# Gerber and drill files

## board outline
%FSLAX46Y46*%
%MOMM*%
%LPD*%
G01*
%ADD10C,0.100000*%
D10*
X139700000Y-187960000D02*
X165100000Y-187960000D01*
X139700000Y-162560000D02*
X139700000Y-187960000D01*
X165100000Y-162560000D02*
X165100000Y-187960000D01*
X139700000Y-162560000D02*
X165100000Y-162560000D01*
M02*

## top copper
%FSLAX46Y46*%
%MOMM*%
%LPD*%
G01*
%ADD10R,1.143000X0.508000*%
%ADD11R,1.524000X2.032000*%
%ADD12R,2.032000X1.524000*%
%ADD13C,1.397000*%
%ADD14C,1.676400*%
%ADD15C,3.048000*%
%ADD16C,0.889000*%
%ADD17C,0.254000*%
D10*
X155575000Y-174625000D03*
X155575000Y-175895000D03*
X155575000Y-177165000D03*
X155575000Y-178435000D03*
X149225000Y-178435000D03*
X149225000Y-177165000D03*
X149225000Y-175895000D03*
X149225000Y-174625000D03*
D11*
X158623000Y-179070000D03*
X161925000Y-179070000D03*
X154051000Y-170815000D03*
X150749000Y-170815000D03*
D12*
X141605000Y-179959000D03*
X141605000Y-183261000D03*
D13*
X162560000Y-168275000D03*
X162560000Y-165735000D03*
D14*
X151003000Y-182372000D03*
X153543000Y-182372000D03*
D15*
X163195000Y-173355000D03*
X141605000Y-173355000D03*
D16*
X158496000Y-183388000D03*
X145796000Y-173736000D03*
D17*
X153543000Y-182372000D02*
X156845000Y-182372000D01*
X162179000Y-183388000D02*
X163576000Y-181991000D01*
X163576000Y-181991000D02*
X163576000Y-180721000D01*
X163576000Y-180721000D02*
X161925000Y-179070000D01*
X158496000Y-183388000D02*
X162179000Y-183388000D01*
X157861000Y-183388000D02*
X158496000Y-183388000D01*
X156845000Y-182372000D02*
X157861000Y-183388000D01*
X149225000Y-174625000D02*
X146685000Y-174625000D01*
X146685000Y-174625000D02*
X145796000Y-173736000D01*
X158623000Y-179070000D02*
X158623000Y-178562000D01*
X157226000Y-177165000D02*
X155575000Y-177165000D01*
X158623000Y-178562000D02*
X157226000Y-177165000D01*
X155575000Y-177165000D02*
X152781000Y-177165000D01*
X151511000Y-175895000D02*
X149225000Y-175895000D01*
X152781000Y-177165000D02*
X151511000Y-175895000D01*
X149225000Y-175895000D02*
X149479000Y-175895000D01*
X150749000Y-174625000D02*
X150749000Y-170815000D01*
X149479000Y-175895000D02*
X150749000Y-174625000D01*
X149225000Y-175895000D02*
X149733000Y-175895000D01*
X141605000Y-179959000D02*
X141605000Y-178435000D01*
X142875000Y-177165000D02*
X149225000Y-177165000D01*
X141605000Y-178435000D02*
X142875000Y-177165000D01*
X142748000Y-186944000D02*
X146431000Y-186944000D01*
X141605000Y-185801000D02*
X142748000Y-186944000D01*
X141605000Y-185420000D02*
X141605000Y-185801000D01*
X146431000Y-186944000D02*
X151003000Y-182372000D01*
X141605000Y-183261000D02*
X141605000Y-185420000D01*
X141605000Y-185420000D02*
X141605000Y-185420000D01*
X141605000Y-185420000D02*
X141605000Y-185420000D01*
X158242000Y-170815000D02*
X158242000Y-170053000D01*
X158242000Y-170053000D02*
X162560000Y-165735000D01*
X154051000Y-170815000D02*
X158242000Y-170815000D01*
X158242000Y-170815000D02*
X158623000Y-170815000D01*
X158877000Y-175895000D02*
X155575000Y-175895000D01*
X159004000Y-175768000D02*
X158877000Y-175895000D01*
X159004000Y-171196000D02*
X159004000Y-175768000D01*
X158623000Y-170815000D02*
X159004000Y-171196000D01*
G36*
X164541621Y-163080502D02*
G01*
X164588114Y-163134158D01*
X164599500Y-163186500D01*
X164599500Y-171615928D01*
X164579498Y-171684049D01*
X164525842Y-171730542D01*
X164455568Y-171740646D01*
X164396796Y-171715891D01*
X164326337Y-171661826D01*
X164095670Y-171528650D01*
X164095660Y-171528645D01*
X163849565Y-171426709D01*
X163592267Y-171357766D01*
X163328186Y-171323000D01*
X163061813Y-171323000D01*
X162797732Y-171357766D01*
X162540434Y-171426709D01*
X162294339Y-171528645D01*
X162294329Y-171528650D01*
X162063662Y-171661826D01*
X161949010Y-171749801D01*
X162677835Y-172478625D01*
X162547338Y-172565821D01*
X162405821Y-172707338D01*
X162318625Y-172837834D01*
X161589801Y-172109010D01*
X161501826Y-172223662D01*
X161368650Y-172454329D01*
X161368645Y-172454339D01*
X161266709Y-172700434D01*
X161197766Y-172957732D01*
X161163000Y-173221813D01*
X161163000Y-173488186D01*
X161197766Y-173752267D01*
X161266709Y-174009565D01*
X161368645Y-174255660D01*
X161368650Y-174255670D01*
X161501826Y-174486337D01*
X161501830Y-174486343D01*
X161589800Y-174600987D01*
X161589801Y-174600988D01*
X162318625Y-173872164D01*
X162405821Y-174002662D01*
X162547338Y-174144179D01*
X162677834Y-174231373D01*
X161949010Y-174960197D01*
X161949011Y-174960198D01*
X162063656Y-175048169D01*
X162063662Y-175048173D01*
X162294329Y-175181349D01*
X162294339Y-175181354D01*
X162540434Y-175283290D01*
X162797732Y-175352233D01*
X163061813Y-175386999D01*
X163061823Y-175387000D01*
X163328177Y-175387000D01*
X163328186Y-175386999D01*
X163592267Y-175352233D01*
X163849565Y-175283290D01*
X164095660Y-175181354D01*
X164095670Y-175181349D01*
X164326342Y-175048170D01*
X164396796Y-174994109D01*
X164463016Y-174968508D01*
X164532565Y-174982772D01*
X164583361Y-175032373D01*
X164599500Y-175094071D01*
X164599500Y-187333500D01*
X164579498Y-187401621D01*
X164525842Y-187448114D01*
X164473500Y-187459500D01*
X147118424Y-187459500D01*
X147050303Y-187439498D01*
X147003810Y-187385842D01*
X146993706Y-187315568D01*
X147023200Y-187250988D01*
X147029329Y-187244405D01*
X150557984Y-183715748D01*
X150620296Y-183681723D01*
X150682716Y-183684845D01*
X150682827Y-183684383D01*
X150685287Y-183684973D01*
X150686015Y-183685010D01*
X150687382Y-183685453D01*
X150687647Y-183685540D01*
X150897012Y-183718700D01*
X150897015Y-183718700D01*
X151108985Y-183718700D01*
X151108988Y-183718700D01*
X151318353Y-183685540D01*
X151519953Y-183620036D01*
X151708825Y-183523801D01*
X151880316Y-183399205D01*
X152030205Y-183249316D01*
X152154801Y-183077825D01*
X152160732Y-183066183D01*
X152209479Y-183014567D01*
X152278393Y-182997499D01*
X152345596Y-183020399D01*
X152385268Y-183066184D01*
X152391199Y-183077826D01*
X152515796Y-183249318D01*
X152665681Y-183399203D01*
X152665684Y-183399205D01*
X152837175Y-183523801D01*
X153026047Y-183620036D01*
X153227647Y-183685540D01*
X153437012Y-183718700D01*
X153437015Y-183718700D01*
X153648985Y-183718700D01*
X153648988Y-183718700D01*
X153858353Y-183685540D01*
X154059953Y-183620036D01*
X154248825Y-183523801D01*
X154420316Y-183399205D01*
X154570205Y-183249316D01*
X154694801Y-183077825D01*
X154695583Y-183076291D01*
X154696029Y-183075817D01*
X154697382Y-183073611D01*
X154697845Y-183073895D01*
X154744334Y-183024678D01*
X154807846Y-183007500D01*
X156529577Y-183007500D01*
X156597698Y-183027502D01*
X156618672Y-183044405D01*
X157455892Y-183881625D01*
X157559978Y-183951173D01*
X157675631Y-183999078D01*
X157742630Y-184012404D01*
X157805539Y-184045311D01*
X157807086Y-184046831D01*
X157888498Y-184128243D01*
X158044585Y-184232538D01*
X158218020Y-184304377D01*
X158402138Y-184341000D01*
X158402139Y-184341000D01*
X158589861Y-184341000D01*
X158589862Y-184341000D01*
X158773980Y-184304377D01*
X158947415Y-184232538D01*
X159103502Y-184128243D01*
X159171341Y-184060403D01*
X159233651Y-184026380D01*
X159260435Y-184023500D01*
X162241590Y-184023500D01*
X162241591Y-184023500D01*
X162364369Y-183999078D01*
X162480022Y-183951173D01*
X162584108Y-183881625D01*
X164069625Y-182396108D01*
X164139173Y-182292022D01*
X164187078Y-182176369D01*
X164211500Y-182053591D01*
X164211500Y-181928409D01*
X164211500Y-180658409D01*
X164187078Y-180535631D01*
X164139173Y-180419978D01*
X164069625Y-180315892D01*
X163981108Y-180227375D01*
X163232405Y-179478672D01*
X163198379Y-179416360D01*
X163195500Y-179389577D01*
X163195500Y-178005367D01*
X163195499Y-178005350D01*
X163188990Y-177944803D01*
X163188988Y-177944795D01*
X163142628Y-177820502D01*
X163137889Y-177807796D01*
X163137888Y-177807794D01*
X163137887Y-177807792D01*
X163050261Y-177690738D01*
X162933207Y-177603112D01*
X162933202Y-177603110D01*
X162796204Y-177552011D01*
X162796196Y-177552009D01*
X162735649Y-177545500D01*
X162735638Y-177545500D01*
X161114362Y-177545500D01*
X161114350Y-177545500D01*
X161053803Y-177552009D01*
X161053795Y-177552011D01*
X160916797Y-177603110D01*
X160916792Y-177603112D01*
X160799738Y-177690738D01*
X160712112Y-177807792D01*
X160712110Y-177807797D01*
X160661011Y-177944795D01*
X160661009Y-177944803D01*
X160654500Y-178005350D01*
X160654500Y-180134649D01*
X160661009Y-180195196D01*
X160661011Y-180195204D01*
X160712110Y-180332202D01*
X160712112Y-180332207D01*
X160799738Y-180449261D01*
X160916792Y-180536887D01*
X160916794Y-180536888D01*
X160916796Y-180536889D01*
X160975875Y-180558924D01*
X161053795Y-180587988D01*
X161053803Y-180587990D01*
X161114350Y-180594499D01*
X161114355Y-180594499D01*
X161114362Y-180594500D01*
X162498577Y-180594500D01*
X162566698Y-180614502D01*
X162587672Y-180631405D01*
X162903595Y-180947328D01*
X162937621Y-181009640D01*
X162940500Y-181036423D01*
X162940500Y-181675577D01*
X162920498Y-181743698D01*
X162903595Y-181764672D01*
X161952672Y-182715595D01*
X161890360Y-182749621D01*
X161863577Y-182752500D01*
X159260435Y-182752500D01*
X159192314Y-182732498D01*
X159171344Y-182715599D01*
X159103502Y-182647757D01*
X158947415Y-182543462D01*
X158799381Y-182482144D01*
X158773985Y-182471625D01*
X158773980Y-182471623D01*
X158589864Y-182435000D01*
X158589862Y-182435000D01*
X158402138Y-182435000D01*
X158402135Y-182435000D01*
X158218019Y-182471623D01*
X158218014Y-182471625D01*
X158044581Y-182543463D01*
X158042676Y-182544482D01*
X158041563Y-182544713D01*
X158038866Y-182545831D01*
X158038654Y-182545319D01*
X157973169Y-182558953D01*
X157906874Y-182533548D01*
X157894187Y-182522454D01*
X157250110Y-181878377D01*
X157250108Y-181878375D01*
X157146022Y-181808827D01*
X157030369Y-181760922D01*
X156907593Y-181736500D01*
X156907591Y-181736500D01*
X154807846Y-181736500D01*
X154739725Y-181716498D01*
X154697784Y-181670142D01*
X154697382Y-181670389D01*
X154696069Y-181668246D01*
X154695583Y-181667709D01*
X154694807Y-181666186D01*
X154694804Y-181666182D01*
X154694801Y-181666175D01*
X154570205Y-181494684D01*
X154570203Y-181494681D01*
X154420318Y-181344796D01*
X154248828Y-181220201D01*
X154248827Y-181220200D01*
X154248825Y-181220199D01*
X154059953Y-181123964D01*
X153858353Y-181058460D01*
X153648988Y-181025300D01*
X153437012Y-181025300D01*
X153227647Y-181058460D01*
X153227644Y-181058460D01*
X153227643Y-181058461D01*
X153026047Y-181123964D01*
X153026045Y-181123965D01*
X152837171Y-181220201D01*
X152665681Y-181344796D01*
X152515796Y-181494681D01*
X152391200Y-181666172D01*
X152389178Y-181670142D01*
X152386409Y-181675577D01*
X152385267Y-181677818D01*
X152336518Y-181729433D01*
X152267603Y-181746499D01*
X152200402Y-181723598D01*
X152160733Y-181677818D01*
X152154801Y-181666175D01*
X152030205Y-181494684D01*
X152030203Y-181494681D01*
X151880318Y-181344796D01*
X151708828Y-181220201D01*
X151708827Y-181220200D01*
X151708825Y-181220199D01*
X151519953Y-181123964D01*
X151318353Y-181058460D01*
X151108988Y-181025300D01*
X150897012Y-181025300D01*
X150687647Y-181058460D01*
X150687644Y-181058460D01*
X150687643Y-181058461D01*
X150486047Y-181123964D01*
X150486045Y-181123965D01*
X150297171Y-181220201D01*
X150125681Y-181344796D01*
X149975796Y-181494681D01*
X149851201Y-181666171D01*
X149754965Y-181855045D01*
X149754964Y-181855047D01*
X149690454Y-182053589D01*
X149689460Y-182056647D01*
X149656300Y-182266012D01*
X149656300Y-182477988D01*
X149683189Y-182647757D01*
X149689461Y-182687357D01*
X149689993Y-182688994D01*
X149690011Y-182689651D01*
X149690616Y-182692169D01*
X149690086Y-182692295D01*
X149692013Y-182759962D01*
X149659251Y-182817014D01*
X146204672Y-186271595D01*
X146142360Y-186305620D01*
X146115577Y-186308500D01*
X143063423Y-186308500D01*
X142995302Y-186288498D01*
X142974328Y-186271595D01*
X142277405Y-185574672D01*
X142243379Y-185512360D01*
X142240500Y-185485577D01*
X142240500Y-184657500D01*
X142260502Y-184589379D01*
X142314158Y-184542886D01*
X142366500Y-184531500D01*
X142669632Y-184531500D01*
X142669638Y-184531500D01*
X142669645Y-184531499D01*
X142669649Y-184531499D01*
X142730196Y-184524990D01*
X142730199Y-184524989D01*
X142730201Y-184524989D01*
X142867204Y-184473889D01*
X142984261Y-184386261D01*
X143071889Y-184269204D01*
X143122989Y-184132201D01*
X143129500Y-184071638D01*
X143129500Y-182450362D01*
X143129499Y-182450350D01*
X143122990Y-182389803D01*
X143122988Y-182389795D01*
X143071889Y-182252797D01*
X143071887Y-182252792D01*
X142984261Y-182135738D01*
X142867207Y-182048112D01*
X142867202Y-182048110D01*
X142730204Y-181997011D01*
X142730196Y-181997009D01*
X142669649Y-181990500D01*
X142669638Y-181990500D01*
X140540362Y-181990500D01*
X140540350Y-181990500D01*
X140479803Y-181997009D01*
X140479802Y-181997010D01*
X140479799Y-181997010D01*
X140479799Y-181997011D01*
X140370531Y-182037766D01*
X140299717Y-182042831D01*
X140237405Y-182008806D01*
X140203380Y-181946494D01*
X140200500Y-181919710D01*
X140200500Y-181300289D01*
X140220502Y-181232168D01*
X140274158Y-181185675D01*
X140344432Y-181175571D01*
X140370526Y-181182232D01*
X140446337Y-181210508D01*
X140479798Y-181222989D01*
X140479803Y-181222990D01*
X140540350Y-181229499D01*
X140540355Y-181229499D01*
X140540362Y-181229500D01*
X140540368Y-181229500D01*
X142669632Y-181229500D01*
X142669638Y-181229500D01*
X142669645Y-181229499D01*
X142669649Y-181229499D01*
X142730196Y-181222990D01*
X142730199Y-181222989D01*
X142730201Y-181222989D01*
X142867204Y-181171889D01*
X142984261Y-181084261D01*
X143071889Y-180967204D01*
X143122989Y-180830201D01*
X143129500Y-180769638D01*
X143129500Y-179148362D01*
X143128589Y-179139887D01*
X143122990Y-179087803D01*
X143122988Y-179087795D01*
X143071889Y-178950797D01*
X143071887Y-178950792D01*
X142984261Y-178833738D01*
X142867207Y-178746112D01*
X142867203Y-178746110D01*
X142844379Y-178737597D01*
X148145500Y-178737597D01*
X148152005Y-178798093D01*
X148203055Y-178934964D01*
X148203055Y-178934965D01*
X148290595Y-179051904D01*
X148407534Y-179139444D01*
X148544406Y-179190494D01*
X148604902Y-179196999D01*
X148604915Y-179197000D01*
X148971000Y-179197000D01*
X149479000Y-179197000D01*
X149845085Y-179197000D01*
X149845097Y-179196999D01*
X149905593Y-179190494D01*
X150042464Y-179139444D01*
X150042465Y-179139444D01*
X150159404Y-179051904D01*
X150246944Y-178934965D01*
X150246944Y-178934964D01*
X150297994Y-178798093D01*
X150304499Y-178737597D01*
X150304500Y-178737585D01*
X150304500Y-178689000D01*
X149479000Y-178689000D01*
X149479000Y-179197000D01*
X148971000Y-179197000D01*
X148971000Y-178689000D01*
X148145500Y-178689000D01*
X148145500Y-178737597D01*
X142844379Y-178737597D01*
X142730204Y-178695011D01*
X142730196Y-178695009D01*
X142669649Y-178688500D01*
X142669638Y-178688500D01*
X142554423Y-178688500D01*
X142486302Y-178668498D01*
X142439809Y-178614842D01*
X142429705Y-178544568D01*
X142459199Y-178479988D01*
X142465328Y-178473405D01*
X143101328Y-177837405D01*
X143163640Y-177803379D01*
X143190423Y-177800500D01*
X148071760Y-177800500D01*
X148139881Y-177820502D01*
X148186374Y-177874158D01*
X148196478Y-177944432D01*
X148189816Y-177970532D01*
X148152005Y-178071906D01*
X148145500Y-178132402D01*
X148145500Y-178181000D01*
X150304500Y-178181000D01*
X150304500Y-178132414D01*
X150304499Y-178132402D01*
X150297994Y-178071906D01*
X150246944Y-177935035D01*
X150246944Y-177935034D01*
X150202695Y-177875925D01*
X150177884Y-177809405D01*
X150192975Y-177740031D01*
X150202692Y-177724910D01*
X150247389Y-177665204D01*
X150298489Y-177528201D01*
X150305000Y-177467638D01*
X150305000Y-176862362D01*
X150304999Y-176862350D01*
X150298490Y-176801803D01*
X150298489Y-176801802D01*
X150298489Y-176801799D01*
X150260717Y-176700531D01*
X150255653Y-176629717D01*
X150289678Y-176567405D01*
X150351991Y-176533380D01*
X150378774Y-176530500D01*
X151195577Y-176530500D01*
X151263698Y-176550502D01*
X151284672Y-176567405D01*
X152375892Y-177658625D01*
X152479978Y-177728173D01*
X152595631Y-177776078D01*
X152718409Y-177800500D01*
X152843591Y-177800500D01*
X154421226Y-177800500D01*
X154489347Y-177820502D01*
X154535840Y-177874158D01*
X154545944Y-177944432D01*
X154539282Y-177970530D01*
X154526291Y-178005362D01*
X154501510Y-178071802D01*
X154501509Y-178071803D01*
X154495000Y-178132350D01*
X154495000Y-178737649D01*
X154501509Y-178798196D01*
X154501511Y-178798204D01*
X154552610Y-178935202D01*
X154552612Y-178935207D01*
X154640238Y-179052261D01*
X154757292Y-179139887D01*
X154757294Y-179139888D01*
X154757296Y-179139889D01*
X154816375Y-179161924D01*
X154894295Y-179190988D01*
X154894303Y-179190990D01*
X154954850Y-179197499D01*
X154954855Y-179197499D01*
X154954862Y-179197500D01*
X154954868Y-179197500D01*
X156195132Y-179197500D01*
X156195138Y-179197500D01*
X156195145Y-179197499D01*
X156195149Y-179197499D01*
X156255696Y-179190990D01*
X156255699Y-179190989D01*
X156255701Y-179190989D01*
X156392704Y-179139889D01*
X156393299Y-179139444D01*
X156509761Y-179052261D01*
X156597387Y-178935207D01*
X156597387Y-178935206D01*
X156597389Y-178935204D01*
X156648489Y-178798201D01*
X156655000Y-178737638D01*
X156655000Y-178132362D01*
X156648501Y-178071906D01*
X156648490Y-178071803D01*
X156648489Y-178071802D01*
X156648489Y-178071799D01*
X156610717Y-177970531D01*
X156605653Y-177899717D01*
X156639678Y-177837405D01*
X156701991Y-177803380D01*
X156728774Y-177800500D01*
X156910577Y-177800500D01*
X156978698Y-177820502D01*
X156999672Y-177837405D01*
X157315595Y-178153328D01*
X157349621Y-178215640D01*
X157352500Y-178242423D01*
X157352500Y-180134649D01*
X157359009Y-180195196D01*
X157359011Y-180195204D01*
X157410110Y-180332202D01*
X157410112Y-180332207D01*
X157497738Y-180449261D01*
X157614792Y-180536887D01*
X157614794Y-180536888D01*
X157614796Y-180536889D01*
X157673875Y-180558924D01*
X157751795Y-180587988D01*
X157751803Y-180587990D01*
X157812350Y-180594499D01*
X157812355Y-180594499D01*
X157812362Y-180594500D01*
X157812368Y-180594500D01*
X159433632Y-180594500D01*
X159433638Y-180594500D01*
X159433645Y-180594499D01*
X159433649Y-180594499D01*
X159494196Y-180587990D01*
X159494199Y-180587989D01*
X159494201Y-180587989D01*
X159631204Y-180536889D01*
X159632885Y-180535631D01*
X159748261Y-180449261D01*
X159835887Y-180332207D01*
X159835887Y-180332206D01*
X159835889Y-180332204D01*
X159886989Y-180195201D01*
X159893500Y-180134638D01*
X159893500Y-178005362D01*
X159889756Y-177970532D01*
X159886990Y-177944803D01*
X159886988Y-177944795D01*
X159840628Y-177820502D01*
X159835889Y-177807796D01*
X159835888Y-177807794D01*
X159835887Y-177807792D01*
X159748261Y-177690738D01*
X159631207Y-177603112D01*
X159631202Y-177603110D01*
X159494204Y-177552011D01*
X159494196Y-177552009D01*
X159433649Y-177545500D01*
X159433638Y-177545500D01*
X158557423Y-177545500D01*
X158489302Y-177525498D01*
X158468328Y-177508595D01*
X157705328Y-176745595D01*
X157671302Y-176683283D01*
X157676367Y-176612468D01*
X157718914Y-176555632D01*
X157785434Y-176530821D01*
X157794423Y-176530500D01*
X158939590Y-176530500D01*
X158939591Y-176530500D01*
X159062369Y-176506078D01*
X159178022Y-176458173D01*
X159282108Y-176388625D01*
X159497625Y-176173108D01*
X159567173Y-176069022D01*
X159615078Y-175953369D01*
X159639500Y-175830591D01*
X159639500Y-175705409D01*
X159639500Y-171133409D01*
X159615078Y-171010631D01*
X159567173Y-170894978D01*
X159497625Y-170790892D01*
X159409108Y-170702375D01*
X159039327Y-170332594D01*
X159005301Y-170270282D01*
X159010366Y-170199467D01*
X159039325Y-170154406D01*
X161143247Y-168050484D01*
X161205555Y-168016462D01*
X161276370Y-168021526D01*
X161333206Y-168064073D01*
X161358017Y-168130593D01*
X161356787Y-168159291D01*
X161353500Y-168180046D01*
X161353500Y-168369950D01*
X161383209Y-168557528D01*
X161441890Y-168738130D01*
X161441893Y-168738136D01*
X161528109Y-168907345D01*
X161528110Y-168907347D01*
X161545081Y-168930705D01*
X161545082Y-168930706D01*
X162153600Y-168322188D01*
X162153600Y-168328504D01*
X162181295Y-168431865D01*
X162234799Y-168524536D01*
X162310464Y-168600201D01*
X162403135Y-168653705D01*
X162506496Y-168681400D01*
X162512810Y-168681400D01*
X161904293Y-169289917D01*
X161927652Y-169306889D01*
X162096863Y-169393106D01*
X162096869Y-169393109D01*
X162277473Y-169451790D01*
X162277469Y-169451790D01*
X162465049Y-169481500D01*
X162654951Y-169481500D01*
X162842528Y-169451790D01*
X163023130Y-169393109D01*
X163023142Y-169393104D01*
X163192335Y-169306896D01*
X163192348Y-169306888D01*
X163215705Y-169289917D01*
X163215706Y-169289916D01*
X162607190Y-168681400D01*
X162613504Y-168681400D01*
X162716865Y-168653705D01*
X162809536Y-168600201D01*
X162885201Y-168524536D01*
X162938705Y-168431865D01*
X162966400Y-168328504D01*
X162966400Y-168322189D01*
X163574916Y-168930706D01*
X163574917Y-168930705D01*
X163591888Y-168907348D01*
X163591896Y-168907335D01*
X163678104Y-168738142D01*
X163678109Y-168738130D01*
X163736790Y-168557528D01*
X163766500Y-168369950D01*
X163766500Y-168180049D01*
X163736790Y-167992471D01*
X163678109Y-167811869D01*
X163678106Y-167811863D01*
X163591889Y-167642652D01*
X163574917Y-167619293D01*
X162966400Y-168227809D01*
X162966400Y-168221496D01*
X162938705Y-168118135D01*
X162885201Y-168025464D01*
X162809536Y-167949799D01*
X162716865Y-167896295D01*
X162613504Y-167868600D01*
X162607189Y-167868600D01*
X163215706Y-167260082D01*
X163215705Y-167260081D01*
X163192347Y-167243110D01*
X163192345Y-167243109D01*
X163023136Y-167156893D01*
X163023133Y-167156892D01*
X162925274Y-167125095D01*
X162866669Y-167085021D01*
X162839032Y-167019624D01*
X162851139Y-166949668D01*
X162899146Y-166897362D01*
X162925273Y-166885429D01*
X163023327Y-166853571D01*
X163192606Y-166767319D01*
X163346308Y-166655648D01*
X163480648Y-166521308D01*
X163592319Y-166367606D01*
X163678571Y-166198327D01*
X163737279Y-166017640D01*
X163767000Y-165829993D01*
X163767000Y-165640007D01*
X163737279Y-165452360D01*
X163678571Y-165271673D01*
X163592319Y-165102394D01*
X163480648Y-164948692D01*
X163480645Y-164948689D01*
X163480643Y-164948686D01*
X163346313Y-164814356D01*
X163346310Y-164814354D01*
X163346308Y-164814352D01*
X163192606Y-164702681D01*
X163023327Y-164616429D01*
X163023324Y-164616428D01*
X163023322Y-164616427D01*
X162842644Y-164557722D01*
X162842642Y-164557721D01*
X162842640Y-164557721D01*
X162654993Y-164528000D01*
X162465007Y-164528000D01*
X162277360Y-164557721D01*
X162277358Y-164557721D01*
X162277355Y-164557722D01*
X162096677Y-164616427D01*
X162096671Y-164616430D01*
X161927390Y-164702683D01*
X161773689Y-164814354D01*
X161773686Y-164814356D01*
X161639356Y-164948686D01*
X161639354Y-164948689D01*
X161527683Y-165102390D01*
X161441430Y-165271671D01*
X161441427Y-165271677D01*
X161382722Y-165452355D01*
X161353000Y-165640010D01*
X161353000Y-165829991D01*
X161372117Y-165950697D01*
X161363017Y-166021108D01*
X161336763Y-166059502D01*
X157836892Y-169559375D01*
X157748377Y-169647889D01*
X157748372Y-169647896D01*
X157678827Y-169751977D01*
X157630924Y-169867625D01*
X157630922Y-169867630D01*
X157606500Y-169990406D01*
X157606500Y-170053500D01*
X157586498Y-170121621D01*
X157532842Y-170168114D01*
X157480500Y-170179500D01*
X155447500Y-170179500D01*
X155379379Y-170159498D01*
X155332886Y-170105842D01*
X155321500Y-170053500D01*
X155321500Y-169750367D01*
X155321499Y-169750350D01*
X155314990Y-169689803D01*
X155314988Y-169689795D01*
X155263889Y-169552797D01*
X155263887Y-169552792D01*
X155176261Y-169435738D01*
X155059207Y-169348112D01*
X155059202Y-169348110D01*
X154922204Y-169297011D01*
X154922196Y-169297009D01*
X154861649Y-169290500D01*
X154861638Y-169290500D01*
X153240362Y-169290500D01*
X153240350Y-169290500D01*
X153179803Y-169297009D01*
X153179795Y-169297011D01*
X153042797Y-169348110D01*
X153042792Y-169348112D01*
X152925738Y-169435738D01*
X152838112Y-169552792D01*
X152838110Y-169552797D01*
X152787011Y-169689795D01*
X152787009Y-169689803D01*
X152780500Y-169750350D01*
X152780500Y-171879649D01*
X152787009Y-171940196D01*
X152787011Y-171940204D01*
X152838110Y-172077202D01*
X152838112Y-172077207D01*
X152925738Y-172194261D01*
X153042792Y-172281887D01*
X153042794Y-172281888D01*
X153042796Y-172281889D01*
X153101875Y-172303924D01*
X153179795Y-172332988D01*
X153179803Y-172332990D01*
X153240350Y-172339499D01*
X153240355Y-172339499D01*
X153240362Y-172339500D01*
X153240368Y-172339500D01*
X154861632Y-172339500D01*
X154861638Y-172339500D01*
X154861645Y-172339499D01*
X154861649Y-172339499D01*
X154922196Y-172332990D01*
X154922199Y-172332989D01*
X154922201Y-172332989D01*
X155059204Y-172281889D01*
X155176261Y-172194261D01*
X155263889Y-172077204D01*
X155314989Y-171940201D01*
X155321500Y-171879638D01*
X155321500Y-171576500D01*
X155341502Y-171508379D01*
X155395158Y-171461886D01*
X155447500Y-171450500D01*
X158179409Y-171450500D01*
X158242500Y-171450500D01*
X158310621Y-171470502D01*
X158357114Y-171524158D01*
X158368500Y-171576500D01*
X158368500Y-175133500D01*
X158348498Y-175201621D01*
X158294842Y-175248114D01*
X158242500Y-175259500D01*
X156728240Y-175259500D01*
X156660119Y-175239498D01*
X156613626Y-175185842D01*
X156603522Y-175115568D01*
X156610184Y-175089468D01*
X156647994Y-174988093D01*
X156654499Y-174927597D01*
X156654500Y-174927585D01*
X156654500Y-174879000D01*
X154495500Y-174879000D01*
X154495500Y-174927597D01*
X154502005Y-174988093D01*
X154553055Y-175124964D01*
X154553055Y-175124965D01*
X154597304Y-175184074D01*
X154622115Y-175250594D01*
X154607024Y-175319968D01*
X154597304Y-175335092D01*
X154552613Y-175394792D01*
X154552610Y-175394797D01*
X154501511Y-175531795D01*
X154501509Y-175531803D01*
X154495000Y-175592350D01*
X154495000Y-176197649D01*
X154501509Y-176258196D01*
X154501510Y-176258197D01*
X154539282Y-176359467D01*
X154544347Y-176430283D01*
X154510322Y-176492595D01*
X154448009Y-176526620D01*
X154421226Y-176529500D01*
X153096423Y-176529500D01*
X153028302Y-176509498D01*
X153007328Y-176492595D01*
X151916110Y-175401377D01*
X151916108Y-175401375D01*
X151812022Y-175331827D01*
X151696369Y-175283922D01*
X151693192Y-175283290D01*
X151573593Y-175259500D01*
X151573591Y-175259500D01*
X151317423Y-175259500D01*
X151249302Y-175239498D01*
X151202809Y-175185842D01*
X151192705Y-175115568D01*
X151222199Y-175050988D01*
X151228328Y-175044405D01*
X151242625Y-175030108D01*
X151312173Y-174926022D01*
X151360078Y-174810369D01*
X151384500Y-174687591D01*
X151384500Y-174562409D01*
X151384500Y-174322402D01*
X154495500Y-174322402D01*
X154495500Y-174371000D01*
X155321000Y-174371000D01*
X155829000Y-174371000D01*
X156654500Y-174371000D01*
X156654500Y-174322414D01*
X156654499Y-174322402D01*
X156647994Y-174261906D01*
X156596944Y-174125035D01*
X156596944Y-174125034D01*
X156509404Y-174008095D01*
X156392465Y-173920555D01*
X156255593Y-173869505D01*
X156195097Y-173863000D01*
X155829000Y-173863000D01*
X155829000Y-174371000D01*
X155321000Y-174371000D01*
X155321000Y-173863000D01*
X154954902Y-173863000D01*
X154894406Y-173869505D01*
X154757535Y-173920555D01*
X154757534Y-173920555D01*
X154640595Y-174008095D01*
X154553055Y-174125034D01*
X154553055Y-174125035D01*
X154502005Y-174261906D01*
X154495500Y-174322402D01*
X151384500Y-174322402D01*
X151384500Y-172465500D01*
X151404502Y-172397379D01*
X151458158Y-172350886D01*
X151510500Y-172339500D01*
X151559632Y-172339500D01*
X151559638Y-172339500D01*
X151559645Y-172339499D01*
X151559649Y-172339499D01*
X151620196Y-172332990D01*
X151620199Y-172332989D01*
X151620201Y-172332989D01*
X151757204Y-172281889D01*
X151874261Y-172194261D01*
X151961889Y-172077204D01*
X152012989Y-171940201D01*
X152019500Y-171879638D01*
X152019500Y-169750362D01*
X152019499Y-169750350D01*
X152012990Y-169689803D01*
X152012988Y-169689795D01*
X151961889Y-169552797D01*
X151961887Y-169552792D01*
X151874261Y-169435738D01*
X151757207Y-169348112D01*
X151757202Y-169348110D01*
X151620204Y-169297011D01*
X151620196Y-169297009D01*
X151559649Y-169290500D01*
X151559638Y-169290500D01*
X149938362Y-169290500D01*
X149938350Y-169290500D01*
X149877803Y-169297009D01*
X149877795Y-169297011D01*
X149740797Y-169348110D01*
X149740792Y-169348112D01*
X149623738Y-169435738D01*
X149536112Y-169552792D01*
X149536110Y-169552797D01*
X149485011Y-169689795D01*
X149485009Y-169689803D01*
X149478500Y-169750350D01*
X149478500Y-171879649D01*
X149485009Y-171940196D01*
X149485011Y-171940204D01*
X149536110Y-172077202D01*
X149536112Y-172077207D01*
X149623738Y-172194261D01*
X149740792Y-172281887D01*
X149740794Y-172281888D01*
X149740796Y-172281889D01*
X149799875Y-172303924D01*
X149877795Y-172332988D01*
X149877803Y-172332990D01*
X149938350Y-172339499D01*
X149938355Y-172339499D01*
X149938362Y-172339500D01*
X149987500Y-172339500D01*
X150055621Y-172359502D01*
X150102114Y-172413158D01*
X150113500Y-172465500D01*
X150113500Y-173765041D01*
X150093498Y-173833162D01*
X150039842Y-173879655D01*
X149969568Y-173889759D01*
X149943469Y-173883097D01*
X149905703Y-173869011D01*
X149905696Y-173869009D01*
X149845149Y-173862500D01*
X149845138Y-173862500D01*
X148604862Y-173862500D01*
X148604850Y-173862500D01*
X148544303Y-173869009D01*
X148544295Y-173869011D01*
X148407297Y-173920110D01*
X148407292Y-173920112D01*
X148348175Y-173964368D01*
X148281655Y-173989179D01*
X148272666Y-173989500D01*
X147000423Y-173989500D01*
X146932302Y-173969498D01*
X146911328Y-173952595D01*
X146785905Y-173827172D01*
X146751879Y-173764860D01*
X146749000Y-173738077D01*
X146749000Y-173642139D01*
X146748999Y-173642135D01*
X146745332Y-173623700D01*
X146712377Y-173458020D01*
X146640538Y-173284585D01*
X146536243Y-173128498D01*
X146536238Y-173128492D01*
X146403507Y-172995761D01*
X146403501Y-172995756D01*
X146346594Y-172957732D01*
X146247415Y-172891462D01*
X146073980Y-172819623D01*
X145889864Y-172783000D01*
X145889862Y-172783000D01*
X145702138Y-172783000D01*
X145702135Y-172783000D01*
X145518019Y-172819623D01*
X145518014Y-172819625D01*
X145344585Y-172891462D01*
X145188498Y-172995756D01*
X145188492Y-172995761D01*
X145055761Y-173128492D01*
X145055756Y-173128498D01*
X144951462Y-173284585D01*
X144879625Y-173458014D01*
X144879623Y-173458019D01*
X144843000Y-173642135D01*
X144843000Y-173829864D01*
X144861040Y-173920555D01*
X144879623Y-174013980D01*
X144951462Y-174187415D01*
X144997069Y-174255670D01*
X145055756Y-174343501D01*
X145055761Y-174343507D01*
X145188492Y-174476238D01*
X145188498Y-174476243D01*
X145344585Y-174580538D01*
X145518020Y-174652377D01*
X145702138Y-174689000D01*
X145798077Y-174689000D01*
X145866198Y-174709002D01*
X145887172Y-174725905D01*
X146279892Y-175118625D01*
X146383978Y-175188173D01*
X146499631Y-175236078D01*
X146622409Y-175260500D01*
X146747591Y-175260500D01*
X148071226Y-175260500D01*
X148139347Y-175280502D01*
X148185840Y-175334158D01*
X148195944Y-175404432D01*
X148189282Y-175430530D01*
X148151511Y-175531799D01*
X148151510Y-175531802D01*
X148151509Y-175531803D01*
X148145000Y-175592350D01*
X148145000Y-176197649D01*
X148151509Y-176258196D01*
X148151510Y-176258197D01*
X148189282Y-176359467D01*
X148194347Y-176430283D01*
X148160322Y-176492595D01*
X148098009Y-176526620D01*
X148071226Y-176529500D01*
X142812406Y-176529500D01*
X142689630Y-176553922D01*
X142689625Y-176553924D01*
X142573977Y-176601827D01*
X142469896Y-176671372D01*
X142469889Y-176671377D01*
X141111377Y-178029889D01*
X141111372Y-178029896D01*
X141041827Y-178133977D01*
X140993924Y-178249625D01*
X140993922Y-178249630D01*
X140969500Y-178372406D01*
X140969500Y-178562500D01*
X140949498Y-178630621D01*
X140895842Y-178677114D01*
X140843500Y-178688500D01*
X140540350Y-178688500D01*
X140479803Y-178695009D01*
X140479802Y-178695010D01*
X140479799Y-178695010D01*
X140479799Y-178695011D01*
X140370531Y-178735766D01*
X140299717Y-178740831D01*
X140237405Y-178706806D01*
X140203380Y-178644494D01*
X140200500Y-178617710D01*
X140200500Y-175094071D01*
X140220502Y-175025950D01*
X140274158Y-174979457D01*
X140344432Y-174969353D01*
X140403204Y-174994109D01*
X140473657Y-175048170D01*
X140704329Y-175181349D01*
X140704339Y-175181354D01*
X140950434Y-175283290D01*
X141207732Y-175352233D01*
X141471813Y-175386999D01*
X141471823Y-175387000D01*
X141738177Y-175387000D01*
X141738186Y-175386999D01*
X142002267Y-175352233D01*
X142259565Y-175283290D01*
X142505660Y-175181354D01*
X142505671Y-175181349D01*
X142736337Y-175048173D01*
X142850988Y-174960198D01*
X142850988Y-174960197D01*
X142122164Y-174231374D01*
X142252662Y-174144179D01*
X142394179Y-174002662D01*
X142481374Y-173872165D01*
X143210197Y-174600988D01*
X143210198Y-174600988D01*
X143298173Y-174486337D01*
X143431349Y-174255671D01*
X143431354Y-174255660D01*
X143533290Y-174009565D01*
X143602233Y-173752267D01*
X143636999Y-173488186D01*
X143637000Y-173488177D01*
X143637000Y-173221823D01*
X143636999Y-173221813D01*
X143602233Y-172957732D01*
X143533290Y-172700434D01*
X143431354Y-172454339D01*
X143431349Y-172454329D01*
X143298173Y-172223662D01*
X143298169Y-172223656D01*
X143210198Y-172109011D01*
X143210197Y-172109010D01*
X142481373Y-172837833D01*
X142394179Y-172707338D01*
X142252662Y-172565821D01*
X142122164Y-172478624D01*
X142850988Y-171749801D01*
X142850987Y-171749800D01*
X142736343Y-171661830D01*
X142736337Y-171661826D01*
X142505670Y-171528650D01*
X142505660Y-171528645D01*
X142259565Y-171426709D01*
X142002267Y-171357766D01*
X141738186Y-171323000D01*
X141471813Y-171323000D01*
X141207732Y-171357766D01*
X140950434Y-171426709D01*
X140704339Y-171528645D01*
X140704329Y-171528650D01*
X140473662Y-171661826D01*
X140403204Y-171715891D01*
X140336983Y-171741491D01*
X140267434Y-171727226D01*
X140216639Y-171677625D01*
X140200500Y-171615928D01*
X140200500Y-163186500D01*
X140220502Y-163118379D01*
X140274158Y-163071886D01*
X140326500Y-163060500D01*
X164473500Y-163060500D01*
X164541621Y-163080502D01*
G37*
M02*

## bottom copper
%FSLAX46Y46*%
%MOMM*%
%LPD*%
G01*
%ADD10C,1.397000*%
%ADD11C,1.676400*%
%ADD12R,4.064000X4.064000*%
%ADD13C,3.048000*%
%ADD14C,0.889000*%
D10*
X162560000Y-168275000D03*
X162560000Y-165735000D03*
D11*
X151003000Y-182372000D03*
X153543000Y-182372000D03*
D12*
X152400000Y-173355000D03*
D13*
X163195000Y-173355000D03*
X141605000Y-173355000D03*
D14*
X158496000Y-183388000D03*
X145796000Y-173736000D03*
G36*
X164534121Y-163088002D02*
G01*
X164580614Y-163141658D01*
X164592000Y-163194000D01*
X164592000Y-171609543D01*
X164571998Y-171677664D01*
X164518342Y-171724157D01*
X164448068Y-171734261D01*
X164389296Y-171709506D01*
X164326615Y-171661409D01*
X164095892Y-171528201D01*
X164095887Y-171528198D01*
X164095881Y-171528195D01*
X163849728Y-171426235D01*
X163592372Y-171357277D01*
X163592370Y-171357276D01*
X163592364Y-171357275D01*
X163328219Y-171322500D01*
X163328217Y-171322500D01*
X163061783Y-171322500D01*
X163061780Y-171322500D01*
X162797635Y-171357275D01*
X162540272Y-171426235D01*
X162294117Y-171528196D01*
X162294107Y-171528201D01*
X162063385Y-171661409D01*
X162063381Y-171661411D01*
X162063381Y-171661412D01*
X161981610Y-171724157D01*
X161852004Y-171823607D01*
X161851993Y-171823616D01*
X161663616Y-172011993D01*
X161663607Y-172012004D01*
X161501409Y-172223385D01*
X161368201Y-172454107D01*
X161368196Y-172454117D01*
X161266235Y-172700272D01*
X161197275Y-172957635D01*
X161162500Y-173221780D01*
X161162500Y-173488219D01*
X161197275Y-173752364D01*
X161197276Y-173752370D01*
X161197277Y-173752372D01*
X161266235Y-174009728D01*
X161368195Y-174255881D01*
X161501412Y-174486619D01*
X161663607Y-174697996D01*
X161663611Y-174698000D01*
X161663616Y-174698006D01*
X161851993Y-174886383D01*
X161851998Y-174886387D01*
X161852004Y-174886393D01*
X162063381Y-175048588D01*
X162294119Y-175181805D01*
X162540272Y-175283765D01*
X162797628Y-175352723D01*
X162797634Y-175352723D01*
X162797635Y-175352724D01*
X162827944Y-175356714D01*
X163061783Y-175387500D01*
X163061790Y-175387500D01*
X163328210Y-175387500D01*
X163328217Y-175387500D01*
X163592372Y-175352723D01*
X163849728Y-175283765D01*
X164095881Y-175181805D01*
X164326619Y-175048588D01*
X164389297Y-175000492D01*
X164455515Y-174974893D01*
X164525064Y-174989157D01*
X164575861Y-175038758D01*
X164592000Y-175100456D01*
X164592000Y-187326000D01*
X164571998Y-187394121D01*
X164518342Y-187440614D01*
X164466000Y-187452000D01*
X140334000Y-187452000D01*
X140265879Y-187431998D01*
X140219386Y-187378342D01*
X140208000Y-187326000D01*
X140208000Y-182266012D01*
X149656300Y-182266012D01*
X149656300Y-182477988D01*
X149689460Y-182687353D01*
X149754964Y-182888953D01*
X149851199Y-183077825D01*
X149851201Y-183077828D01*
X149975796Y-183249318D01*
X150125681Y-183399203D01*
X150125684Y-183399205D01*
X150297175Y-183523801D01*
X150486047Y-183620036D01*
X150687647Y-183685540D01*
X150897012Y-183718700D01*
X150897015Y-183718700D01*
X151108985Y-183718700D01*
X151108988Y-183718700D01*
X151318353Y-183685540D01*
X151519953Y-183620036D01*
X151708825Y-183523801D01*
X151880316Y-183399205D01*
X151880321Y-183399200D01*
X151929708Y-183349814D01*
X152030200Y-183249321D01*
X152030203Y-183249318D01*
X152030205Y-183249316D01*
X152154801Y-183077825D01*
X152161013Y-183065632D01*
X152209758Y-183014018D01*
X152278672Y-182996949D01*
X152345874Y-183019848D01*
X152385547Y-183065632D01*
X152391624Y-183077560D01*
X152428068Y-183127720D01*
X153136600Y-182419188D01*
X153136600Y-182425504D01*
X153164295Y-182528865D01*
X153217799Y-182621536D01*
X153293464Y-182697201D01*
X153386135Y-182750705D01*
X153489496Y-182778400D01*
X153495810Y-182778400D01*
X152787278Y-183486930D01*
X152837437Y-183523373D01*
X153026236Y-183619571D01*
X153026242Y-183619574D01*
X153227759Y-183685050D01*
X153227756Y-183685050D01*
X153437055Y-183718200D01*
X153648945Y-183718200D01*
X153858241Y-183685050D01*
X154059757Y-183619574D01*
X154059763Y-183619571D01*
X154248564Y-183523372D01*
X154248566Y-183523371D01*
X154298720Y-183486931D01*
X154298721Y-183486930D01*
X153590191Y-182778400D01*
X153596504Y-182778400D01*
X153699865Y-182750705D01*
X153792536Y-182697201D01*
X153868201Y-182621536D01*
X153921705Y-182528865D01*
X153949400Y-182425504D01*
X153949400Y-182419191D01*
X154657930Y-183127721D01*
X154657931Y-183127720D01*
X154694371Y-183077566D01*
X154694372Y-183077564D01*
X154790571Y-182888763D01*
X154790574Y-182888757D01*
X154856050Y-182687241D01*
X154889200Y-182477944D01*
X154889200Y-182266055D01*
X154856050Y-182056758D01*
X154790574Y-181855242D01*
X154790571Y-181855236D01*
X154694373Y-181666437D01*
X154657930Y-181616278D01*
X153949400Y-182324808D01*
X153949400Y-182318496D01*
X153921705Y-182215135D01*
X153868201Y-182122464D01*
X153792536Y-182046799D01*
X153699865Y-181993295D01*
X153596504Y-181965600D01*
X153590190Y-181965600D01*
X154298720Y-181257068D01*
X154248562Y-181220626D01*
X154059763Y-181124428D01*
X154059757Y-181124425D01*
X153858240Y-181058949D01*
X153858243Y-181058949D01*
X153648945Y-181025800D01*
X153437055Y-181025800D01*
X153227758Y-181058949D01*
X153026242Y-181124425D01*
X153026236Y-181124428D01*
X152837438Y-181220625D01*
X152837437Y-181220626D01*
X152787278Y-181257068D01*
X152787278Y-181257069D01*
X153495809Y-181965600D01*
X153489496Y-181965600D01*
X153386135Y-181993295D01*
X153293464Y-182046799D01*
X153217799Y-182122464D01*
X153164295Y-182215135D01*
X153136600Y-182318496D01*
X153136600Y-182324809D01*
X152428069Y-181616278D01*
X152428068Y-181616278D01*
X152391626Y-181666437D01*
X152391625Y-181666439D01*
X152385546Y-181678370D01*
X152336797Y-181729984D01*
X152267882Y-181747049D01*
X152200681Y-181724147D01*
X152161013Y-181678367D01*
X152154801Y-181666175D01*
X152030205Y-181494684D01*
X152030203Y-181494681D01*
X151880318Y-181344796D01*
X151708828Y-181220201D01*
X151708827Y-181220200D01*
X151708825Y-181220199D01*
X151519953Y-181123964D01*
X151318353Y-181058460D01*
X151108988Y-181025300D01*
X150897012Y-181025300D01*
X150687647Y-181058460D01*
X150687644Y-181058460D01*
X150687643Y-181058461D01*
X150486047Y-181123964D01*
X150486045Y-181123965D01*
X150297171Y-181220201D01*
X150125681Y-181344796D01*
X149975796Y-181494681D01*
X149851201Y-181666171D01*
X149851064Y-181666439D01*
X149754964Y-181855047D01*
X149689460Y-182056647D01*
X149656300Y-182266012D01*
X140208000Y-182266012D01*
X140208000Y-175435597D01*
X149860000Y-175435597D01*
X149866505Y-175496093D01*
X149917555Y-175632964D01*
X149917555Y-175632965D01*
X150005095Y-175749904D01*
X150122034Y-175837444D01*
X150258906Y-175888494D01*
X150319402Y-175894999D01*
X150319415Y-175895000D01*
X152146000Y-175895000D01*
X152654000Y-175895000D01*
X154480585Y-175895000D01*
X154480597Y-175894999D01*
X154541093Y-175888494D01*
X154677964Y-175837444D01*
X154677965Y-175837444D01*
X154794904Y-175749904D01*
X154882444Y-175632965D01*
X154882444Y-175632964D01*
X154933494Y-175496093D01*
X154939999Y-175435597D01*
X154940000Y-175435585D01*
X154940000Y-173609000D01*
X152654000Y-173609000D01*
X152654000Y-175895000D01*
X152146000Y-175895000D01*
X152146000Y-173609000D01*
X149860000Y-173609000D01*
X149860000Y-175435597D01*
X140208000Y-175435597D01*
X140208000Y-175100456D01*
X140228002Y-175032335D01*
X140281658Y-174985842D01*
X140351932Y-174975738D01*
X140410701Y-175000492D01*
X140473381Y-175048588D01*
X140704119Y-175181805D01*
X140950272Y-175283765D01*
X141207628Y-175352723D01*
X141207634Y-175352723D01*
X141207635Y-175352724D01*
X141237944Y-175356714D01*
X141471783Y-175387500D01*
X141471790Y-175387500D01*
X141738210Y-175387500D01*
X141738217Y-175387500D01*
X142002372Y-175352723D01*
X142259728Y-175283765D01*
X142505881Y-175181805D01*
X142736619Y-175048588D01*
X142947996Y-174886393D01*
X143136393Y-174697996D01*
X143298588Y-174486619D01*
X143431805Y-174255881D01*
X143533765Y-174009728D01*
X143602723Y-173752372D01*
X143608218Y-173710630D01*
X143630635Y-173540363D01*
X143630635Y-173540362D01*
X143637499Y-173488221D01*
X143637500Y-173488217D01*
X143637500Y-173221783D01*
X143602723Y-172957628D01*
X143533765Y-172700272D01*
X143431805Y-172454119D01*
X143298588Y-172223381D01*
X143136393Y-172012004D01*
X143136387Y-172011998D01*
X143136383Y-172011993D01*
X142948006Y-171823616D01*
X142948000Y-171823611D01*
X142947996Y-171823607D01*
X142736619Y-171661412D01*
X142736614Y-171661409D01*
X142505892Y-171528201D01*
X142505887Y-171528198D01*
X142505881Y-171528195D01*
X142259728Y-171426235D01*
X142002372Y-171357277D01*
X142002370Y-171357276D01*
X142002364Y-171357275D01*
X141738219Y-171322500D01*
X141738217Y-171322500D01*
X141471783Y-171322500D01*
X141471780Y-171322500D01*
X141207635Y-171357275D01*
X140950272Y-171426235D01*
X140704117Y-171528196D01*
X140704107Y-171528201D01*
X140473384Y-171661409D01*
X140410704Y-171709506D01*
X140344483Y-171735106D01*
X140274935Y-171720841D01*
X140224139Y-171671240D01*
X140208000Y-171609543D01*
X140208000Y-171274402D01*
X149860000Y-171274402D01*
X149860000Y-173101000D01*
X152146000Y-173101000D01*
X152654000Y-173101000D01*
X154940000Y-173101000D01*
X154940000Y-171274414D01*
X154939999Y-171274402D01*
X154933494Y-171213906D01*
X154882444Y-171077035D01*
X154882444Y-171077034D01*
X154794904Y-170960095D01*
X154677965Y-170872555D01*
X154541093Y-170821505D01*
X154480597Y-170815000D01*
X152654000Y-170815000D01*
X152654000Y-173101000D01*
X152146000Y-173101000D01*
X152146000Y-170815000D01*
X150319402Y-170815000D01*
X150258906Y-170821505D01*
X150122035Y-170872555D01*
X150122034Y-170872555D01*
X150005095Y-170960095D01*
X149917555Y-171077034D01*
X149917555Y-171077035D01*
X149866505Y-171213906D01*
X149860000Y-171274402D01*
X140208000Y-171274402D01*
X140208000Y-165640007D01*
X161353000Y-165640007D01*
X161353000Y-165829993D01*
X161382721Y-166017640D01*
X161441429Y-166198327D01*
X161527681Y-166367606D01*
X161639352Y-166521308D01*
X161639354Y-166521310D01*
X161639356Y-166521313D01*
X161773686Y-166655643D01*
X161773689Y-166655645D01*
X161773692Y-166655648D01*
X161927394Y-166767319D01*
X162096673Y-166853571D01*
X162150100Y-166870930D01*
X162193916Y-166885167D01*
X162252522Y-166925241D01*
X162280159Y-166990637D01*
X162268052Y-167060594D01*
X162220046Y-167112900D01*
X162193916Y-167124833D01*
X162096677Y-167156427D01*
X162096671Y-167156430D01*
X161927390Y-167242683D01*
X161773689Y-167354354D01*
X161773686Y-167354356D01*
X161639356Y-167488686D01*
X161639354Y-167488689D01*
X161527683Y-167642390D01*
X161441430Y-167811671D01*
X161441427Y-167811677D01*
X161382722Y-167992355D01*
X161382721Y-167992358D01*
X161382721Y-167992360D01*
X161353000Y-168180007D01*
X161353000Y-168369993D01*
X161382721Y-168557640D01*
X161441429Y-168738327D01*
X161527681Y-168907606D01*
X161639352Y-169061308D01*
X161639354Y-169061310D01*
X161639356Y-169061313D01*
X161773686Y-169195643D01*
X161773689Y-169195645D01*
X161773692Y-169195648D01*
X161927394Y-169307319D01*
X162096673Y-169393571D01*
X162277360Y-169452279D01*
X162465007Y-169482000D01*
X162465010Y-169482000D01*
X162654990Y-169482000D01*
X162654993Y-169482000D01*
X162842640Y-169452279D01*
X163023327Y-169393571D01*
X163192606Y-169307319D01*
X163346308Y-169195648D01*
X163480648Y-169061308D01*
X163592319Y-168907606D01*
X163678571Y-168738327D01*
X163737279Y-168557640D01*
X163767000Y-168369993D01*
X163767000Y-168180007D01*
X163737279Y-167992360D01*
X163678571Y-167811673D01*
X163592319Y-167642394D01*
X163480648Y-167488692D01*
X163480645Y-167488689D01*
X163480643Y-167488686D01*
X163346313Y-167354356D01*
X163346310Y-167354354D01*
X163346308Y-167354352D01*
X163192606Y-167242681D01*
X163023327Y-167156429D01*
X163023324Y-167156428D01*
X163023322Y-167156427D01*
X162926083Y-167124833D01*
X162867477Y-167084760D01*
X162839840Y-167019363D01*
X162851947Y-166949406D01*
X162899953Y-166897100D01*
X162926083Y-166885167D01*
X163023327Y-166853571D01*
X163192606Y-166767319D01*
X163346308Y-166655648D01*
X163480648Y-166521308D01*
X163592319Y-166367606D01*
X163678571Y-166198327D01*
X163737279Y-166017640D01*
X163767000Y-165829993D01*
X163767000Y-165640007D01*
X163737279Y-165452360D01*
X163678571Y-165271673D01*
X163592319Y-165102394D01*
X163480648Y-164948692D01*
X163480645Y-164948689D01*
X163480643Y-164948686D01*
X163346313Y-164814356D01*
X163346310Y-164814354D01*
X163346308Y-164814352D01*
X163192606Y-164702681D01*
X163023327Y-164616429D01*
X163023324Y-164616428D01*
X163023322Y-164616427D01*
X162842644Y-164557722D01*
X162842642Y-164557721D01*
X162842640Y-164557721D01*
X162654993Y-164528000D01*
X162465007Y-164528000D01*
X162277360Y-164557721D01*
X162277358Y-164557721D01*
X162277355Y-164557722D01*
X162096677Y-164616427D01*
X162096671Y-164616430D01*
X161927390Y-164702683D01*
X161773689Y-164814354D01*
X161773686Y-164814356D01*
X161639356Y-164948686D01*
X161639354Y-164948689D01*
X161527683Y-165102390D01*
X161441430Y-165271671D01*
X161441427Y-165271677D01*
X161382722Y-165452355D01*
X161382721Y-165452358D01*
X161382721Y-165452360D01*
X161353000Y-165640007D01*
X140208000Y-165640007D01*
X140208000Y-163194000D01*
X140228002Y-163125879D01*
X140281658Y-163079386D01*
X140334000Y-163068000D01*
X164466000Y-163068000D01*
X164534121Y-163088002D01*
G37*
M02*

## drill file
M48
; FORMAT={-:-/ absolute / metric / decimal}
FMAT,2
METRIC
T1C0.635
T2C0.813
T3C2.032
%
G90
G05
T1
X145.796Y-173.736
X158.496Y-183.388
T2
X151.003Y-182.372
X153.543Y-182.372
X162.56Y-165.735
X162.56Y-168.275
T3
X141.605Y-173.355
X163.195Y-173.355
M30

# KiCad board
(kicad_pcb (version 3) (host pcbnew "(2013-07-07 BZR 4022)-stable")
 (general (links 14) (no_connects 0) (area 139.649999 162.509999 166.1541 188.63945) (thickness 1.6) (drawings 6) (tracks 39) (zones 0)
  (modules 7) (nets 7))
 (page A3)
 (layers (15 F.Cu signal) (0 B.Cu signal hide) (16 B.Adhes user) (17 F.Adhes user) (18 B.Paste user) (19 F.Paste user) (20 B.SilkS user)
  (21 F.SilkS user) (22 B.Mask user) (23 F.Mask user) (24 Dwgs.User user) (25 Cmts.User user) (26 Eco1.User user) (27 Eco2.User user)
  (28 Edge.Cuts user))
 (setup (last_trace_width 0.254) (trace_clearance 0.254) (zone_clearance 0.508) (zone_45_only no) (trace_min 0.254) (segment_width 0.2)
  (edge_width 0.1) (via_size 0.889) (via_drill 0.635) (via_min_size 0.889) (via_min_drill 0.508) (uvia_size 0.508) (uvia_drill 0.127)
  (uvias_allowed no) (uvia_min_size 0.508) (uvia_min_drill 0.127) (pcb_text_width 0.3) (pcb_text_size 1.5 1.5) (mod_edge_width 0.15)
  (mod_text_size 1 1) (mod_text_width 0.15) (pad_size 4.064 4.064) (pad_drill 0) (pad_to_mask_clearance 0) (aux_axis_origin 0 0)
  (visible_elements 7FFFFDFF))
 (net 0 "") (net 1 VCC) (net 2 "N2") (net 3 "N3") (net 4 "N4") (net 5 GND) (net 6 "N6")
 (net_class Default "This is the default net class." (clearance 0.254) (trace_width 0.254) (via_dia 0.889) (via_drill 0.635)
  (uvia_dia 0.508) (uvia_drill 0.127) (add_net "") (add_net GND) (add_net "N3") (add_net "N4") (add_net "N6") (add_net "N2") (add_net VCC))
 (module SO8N (layer F.Cu) (at 152.4 176.53 270)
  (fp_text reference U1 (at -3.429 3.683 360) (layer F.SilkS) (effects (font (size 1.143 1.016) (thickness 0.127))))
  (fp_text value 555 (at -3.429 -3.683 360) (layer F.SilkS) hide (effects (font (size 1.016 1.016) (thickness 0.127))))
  (pad 8 smd rect (at -1.905 -3.175 270) (size 0.508 1.143) (layers F.Cu F.Paste F.Mask) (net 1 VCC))
  (pad 7 smd rect (at -0.635 -3.175 270) (size 0.508 1.143) (layers F.Cu F.Paste F.Mask) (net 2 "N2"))
  (pad 6 smd rect (at 0.635 -3.175 270) (size 0.508 1.143) (layers F.Cu F.Paste F.Mask) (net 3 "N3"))
  (pad 5 smd rect (at 1.905 -3.175 270) (size 0.508 1.143) (layers F.Cu F.Paste F.Mask))
  (pad 4 smd rect (at 1.905 3.175 270) (size 0.508 1.143) (layers F.Cu F.Paste F.Mask) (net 1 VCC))
  (pad 3 smd rect (at 0.635 3.175 270) (size 0.508 1.143) (layers F.Cu F.Paste F.Mask) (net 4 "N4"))
  (pad 2 smd rect (at -0.635 3.175 270) (size 0.508 1.143) (layers F.Cu F.Paste F.Mask) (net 3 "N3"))
  (pad 1 smd rect (at -1.905 3.175 270) (size 0.508 1.143) (layers F.Cu F.Paste F.Mask) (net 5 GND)))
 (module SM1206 (layer F.Cu) (at 160.274 179.07)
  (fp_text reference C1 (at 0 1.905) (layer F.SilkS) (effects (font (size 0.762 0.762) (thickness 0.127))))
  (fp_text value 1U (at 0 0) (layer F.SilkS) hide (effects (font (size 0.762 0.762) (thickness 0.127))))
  (pad 1 smd rect (at -1.651 0) (size 1.524 2.032) (layers F.Cu F.Paste F.Mask) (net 3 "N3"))
  (pad 2 smd rect (at 1.651 0) (size 1.524 2.032) (layers F.Cu F.Paste F.Mask) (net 5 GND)))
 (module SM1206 (layer F.Cu) (at 152.4 170.815 180)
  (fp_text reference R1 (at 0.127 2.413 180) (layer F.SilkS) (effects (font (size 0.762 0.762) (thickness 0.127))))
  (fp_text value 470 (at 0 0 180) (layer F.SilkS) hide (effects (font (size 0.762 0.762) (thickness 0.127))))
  (pad 1 smd rect (at -1.651 0 180) (size 1.524 2.032) (layers F.Cu F.Paste F.Mask) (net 2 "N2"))
  (pad 2 smd rect (at 1.651 0 180) (size 1.524 2.032) (layers F.Cu F.Paste F.Mask) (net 3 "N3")))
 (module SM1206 (layer F.Cu) (at 141.605 181.61 270)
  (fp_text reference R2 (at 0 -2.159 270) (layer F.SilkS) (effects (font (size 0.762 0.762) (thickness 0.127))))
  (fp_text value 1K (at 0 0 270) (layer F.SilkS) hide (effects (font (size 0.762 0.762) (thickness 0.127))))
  (pad 1 smd rect (at -1.651 0 270) (size 1.524 2.032) (layers F.Cu F.Paste F.Mask) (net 4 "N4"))
  (pad 2 smd rect (at 1.651 0 270) (size 1.524 2.032) (layers F.Cu F.Paste F.Mask) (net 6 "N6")))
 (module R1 (layer F.Cu) (at 162.56 167.005 90) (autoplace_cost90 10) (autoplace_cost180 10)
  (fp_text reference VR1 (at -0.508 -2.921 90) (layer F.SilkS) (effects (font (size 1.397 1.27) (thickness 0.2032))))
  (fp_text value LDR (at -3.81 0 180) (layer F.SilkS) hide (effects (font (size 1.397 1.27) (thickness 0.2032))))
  (pad 1 thru_hole circle (at -1.27 0 90) (size 1.397 1.397) (drill 0.8128) (layers *.Cu *.Mask F.SilkS) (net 1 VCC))
  (pad 2 thru_hole circle (at 1.27 0 90) (size 1.397 1.397) (drill 0.8128) (layers *.Cu *.Mask F.SilkS) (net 2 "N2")))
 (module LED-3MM (layer F.Cu) (at 152.273 182.372)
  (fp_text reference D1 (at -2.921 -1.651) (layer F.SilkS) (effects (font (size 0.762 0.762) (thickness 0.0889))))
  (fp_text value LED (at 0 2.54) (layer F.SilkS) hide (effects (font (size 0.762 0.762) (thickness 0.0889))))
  (pad 1 thru_hole circle (at -1.27 0) (size 1.6764 1.6764) (drill 0.8128) (layers *.Cu *.Mask F.SilkS) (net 6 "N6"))
  (pad 2 thru_hole circle (at 1.27 0) (size 1.6764 1.6764) (drill 0.8128) (layers *.Cu *.Mask F.SilkS) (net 5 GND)))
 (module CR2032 (layer B.Cu) (at 152.4 173.355 180)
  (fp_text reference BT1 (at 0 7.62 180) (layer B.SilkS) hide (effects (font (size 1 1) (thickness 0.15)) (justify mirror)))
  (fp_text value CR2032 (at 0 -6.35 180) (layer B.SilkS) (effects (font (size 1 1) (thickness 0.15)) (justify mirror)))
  (pad 2 smd rect (at 0 0 180) (size 4.064 4.064) (layers B.Cu B.Paste B.Mask) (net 5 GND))
  (pad 1 thru_hole circle (at -10.795 0 180) (size 3.048 3.048) (drill 2.032) (layers *.Cu *.Mask B.SilkS) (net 1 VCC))
  (pad 1 thru_hole circle (at 10.795 0 180) (size 3.048 3.048) (drill 2.032) (layers *.Cu *.Mask B.SilkS) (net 1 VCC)))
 (gr_line (start 139.7 187.96) (end 165.1 187.96) (angle 90) (layer Edge.Cuts) (width 0.1))
 (gr_line (start 139.7 162.56) (end 139.7 187.96) (angle 90) (layer Edge.Cuts) (width 0.1))
 (gr_line (start 165.1 162.56) (end 165.1 187.96) (angle 90) (layer Edge.Cuts) (width 0.1))
 (gr_line (start 139.7 162.56) (end 165.1 162.56) (angle 90) (layer Edge.Cuts) (width 0.1))
 (segment (start 153.543 182.372) (end 156.845 182.372) (width 0.254) (layer F.Cu) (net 5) (status 400000))
 (segment (start 162.179 183.388) (end 163.576 181.991) (width 0.254) (layer F.Cu) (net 5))
 (segment (start 163.576 181.991) (end 163.576 180.721) (width 0.254) (layer F.Cu) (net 5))
 (segment (start 163.576 180.721) (end 161.925 179.07) (width 0.254) (layer F.Cu) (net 5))
 (via (at 158.496 183.388) (size 0.889) (layers F.Cu B.Cu) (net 5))
 (segment (start 158.496 183.388) (end 162.179 183.388) (width 0.254) (layer F.Cu) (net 5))
 (segment (start 157.861 183.388) (end 158.496 183.388) (width 0.254) (layer F.Cu) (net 5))
 (segment (start 156.845 182.372) (end 157.861 183.388) (width 0.254) (layer F.Cu) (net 5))
 (segment (start 149.225 174.625) (end 146.685 174.625) (width 0.254) (layer F.Cu) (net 5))
 (via (at 145.796 173.736) (size 0.889) (layers F.Cu B.Cu) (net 5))
 (segment (start 146.685 174.625) (end 145.796 173.736) (width 0.254) (layer F.Cu) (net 5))
 (segment (start 158.623 179.07) (end 158.623 178.562) (width 0.254) (layer F.Cu) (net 3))
 (segment (start 157.226 177.165) (end 155.575 177.165) (width 0.254) (layer F.Cu) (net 3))
 (segment (start 158.623 178.562) (end 157.226 177.165) (width 0.254) (layer F.Cu) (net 3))
 (segment (start 155.575 177.165) (end 152.781 177.165) (width 0.254) (layer F.Cu) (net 3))
 (segment (start 151.511 175.895) (end 149.225 175.895) (width 0.254) (layer F.Cu) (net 3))
 (segment (start 152.781 177.165) (end 151.511 175.895) (width 0.254) (layer F.Cu) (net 3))
 (segment (start 149.225 175.895) (end 149.479 175.895) (width 0.254) (layer F.Cu) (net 3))
 (segment (start 150.749 174.625) (end 150.749 170.815) (width 0.254) (layer F.Cu) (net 3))
 (segment (start 149.479 175.895) (end 150.749 174.625) (width 0.254) (layer F.Cu) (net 3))
 (segment (start 149.225 175.895) (end 149.733 175.895) (width 0.254) (layer F.Cu) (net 3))
 (segment (start 141.605 179.959) (end 141.605 178.435) (width 0.254) (layer F.Cu) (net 4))
 (segment (start 142.875 177.165) (end 149.225 177.165) (width 0.254) (layer F.Cu) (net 4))
 (segment (start 141.605 178.435) (end 142.875 177.165) (width 0.254) (layer F.Cu) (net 4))
 (segment (start 142.748 186.944) (end 146.431 186.944) (width 0.254) (layer F.Cu) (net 6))
 (segment (start 141.605 185.801) (end 142.748 186.944) (width 0.254) (layer F.Cu) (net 6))
 (segment (start 141.605 185.42) (end 141.605 185.801) (width 0.254) (layer F.Cu) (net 6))
 (segment (start 146.431 186.944) (end 151.003 182.372) (width 0.254) (layer F.Cu) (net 6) (status 800000))
 (segment (start 141.605 183.261) (end 141.605 185.42) (width 0.254) (layer F.Cu) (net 6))
 (segment (start 141.605 185.42) (end 141.605 185.42) (width 0.254) (layer F.Cu) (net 6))
 (segment (start 141.605 185.42) (end 141.605 185.42) (width 0.254) (layer F.Cu) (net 6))
 (segment (start 158.242 170.815) (end 158.242 170.053) (width 0.254) (layer F.Cu) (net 2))
 (segment (start 158.242 170.053) (end 162.56 165.735) (width 0.254) (layer F.Cu) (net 2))
 (segment (start 154.051 170.815) (end 158.242 170.815) (width 0.254) (layer F.Cu) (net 2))
 (segment (start 158.242 170.815) (end 158.623 170.815) (width 0.254) (layer F.Cu) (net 2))
 (segment (start 158.877 175.895) (end 155.575 175.895) (width 0.254) (layer F.Cu) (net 2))
 (segment (start 159.004 175.768) (end 158.877 175.895) (width 0.254) (layer F.Cu) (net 2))
 (segment (start 159.004 171.196) (end 159.004 175.768) (width 0.254) (layer F.Cu) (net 2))
 (segment (start 158.623 170.815) (end 159.004 171.196) (width 0.254) (layer F.Cu) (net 2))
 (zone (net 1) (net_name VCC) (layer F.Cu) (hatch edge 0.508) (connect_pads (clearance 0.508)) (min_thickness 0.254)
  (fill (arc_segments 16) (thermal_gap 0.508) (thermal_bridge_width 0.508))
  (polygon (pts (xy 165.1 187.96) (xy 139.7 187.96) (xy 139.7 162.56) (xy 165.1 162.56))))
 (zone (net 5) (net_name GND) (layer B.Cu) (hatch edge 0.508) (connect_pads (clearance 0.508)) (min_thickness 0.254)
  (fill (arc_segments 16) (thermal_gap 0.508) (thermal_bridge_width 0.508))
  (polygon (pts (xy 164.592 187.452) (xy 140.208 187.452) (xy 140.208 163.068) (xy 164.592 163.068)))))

